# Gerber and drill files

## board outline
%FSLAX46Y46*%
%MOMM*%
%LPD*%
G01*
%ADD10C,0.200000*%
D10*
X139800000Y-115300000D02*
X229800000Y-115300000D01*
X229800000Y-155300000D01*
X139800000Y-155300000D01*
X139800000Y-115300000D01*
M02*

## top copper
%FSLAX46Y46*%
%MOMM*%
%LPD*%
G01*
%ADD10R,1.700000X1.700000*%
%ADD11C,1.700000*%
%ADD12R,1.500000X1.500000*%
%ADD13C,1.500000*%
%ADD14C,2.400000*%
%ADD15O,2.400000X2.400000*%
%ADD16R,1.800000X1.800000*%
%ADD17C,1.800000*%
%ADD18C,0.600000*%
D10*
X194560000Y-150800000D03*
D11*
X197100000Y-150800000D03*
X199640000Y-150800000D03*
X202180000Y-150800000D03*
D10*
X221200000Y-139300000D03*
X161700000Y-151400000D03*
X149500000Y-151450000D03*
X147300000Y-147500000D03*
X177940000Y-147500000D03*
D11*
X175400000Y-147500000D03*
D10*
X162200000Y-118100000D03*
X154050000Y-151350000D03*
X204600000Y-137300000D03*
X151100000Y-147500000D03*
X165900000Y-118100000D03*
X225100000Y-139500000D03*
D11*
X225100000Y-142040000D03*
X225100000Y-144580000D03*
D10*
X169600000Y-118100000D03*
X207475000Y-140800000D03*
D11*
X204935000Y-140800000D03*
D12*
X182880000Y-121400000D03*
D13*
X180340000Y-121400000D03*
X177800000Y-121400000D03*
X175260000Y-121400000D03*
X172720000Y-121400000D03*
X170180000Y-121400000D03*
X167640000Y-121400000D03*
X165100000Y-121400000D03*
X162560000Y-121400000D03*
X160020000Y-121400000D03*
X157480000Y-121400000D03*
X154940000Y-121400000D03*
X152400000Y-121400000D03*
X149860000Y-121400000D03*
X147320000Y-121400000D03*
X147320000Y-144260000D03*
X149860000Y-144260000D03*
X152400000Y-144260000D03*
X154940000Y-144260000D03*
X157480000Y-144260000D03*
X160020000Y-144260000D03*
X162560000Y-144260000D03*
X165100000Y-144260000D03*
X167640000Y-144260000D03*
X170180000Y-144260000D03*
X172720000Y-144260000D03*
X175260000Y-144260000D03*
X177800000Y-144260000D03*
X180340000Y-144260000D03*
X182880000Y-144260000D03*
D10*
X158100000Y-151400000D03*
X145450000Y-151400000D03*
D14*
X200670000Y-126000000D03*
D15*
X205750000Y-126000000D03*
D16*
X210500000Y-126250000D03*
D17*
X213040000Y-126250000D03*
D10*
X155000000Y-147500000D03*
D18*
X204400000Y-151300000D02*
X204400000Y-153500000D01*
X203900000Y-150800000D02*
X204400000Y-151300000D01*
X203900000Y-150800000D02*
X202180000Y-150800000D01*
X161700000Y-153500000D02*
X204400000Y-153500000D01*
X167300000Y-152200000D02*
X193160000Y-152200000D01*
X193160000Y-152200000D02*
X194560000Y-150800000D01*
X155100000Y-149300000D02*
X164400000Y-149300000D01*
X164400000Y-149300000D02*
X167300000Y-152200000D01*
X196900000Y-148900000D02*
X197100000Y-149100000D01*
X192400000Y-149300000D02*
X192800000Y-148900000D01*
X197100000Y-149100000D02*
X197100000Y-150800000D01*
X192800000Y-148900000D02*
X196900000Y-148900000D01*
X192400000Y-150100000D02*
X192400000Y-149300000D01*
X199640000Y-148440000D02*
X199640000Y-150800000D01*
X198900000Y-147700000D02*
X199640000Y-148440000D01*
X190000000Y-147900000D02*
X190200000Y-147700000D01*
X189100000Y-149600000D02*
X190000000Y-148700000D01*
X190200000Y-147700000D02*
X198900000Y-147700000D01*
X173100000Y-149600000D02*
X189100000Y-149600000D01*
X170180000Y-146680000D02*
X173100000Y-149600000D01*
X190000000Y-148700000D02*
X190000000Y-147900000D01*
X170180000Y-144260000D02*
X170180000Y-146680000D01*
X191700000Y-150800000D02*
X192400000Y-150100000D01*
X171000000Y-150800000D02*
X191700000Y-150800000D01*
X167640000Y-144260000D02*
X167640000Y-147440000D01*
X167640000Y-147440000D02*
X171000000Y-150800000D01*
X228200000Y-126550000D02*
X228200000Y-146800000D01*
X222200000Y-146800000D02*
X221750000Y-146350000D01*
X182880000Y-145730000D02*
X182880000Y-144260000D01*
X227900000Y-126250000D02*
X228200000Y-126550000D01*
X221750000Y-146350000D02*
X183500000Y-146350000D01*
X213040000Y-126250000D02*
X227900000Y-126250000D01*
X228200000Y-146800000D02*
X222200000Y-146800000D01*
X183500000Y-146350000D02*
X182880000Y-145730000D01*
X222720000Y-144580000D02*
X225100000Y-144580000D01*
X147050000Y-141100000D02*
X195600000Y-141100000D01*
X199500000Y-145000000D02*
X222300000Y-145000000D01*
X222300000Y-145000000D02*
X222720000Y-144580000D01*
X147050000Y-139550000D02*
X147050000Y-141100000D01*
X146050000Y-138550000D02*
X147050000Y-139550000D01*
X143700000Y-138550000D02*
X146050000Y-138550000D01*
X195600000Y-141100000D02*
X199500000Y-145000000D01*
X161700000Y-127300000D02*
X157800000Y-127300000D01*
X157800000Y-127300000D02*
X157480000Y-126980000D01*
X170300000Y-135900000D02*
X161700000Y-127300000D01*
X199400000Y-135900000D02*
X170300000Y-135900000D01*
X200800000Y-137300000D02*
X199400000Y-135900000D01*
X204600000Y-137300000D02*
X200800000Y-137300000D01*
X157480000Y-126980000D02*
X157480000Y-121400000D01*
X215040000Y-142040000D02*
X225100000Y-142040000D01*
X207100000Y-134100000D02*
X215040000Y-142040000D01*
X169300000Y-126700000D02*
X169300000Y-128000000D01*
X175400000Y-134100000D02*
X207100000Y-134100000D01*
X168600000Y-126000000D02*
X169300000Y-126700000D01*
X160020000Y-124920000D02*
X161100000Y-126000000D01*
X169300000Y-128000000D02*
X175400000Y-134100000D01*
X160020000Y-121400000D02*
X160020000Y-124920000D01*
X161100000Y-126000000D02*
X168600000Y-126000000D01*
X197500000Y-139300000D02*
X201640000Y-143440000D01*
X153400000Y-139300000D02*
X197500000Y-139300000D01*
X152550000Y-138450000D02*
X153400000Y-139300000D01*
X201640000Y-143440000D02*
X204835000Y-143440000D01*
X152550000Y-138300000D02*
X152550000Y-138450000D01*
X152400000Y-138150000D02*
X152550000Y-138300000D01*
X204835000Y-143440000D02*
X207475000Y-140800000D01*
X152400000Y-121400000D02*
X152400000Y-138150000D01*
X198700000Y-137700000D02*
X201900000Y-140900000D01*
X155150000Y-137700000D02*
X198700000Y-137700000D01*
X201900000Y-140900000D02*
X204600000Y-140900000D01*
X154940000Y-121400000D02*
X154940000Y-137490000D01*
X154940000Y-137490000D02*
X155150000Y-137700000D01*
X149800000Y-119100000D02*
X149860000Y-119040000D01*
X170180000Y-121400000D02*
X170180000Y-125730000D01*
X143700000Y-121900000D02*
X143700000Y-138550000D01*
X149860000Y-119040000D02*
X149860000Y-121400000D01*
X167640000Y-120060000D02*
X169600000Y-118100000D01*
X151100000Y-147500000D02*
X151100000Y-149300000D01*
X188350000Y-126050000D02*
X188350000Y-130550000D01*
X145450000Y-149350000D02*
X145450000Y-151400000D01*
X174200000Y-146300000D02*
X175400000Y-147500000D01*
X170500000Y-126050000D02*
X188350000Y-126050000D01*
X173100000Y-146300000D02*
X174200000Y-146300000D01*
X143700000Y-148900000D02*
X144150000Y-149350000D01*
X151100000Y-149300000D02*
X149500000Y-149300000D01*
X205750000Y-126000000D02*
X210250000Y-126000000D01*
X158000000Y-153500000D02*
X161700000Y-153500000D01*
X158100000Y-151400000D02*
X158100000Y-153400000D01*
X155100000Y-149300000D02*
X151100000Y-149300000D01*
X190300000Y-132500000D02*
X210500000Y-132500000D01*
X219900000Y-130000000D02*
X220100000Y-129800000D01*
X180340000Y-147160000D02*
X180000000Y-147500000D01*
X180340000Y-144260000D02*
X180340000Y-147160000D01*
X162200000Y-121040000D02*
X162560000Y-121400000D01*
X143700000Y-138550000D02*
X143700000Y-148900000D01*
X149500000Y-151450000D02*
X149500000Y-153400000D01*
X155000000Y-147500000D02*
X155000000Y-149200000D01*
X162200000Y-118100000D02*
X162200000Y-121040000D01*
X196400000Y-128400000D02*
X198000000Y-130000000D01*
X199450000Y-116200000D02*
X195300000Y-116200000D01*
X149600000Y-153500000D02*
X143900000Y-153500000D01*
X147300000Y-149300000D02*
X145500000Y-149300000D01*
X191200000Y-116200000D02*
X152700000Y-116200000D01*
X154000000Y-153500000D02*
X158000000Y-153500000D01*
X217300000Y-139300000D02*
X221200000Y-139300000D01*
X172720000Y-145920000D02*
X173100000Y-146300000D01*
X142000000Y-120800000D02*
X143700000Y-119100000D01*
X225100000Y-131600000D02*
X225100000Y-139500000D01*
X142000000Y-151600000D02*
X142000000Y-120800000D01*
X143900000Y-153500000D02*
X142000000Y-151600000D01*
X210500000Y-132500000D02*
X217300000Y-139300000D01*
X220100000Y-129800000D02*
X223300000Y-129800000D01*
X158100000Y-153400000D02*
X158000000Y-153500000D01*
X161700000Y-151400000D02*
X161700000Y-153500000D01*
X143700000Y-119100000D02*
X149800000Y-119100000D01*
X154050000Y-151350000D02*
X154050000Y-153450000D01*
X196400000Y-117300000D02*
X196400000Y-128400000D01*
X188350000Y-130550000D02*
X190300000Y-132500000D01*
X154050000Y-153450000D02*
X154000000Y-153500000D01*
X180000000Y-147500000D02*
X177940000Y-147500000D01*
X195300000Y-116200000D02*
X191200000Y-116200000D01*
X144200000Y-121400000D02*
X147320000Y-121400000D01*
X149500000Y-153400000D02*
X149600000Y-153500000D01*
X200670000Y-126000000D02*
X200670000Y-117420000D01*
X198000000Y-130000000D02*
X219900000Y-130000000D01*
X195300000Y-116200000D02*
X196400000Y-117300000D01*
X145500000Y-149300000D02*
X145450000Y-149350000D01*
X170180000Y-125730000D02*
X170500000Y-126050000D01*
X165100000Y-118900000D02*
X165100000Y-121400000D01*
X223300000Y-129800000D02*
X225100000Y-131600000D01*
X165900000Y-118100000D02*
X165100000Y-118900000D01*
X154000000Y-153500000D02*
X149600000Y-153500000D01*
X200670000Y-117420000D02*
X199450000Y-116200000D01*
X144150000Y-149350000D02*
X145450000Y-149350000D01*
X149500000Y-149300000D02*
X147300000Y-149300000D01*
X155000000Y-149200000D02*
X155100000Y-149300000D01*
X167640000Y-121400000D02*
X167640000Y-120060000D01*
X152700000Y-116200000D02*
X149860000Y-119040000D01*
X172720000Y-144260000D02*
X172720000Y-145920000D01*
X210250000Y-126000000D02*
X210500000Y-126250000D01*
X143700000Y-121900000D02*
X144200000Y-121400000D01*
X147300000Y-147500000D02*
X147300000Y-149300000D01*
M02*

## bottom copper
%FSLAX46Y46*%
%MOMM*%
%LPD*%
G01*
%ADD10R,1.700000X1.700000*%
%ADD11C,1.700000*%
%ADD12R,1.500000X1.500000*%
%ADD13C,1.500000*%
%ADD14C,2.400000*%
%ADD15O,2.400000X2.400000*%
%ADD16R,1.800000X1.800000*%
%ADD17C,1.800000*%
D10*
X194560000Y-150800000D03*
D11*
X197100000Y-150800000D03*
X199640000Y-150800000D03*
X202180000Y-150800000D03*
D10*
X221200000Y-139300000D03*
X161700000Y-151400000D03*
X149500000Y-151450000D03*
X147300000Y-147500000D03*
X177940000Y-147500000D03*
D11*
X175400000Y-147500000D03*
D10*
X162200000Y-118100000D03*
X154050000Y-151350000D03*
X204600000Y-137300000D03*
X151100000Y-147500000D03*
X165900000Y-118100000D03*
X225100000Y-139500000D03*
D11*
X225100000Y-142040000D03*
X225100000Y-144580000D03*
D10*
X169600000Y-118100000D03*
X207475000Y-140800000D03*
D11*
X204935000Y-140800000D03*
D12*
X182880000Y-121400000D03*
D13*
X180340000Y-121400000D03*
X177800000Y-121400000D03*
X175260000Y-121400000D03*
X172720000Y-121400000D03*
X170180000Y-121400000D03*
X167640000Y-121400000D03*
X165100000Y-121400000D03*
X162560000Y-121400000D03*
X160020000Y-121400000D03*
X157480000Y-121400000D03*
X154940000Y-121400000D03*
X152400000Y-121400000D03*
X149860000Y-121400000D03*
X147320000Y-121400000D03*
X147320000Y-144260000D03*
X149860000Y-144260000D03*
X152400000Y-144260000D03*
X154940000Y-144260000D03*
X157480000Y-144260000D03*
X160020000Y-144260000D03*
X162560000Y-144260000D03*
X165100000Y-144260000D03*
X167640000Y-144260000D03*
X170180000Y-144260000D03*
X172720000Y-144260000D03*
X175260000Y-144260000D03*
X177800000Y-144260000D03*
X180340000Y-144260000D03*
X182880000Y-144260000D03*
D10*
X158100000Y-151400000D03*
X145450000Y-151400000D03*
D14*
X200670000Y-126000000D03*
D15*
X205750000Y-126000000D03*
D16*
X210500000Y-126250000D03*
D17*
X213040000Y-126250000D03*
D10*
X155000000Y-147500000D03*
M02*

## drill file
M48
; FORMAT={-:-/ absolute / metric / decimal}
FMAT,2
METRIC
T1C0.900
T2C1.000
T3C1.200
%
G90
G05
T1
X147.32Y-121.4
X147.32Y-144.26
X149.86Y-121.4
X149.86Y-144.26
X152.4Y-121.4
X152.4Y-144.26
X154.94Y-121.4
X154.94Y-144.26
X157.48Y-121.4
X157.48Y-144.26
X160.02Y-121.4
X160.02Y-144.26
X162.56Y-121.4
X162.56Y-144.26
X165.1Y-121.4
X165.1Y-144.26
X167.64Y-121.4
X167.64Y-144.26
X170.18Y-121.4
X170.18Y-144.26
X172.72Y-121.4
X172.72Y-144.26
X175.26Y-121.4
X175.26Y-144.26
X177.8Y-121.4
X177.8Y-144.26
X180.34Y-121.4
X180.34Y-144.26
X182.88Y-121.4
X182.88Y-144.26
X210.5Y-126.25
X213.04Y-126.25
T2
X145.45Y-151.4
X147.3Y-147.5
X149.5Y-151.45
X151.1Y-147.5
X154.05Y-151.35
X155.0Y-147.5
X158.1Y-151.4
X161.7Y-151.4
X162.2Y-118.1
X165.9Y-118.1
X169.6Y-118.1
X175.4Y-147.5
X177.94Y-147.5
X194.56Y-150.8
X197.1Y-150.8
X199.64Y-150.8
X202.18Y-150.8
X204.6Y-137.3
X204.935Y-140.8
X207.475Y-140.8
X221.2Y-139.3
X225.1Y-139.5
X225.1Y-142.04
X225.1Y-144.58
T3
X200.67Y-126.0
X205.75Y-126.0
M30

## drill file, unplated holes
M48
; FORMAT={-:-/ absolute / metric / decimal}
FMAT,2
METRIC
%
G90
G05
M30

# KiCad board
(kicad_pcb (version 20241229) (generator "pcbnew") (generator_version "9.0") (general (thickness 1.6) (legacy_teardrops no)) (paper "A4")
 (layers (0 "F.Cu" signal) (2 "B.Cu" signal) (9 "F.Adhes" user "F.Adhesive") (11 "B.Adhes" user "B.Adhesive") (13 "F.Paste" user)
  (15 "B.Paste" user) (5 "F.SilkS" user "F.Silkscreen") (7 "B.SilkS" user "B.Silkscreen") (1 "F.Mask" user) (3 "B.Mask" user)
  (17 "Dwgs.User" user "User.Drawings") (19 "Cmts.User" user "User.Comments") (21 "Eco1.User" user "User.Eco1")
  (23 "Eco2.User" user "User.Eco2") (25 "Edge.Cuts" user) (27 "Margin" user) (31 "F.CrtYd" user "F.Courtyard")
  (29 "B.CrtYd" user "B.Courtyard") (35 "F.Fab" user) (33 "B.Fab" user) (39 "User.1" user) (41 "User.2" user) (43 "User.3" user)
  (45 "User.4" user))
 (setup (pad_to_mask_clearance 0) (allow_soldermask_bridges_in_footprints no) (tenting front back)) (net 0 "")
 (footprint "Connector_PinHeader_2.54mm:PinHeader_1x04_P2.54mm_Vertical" (layer "F.Cu") (at 194.56 150.8 90)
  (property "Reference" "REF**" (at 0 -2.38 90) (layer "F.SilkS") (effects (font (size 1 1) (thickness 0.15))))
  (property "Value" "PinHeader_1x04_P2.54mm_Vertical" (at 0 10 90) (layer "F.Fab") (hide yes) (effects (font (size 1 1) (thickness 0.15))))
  (pad "1" thru_hole rect (at 0 0 90) (size 1.7 1.7) (drill 1) (layers "*.Cu" "*.Mask") (remove_unused_layers no))
  (pad "2" thru_hole circle (at 0 2.54 90) (size 1.7 1.7) (drill 1) (layers "*.Cu" "*.Mask") (remove_unused_layers no))
  (pad "3" thru_hole circle (at 0 5.08 90) (size 1.7 1.7) (drill 1) (layers "*.Cu" "*.Mask") (remove_unused_layers no))
  (pad "4" thru_hole circle (at 0 7.62 90) (size 1.7 1.7) (drill 1) (layers "*.Cu" "*.Mask") (remove_unused_layers no)))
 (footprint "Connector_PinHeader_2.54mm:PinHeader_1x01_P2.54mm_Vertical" (layer "F.Cu") (at 221.2 139.3 90)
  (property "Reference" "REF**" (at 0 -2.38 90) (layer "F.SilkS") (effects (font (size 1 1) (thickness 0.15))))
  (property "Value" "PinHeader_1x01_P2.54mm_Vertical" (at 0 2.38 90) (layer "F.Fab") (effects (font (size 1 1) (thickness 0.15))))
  (pad "1" thru_hole rect (at 0 0 90) (size 1.7 1.7) (drill 1) (layers "*.Cu" "*.Mask") (remove_unused_layers no)))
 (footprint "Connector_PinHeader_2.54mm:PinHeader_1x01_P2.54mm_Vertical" (layer "F.Cu") (at 161.7 151.4)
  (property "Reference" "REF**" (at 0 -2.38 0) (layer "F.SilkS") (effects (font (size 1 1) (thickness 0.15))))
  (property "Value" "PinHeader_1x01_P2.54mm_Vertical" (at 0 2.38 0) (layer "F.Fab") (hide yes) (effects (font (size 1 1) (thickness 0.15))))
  (pad "1" thru_hole rect (at 0 0) (size 1.7 1.7) (drill 1) (layers "*.Cu" "*.Mask") (remove_unused_layers no)))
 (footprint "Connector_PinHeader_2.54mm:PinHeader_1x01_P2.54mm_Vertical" (layer "F.Cu") (at 149.5 151.45)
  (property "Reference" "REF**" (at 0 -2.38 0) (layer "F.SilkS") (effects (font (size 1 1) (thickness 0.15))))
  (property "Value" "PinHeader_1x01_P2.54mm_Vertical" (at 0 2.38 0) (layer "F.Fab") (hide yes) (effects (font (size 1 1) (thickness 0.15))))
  (pad "1" thru_hole rect (at 0 0) (size 1.7 1.7) (drill 1) (layers "*.Cu" "*.Mask") (remove_unused_layers no)))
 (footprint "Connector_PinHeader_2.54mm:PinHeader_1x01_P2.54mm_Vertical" (layer "F.Cu") (at 147.3 147.5)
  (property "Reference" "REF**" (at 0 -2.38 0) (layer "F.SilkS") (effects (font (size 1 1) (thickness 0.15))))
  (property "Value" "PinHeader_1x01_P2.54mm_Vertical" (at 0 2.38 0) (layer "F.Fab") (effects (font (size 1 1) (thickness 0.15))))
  (pad "1" thru_hole rect (at 0 0) (size 1.7 1.7) (drill 1) (layers "*.Cu" "*.Mask") (remove_unused_layers no)))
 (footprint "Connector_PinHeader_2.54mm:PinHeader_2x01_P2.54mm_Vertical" (layer "F.Cu") (at 177.94 147.5 180)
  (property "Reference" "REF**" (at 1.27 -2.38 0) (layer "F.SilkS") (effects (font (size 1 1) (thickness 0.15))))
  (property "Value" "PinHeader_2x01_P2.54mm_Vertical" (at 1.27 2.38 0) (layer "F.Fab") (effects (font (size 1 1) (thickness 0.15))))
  (pad "1" thru_hole rect (at 0 0 180) (size 1.7 1.7) (drill 1) (layers "*.Cu" "*.Mask") (remove_unused_layers no))
  (pad "2" thru_hole circle (at 2.54 0 180) (size 1.7 1.7) (drill 1) (layers "*.Cu" "*.Mask") (remove_unused_layers no)))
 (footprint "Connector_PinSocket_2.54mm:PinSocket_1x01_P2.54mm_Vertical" (layer "F.Cu") (at 162.2 118.1)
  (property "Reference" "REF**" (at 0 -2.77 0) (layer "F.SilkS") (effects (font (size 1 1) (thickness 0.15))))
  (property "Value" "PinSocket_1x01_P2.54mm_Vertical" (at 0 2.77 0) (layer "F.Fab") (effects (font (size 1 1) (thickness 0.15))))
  (pad "1" thru_hole rect (at 0 0) (size 1.7 1.7) (drill 1) (layers "*.Cu" "*.Mask") (remove_unused_layers no)))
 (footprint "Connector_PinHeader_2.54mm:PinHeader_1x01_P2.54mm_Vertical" (layer "F.Cu") (at 154.05 151.35 -90)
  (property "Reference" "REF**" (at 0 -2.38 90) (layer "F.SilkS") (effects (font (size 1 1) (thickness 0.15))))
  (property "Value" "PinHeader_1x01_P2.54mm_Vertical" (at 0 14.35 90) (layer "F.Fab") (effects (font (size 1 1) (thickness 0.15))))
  (pad "1" thru_hole rect (at 0 0 270) (size 1.7 1.7) (drill 1) (layers "*.Cu" "*.Mask") (remove_unused_layers no)))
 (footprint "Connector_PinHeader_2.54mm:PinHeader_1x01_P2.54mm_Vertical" (layer "F.Cu") (at 204.6 137.3 90)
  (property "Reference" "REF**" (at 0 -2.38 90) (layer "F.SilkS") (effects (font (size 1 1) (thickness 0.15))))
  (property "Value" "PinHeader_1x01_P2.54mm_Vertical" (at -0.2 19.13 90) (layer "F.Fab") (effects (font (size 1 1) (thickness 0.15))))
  (pad "1" thru_hole rect (at 0 0 90) (size 1.7 1.7) (drill 1) (layers "*.Cu" "*.Mask") (remove_unused_layers no)))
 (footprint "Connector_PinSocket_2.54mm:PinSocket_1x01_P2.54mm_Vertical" (layer "F.Cu") (at 151.1 147.5)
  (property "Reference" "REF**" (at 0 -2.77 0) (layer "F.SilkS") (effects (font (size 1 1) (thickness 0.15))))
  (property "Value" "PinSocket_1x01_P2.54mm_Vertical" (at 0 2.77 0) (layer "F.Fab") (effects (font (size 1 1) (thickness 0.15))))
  (pad "1" thru_hole rect (at 0 0) (size 1.7 1.7) (drill 1) (layers "*.Cu" "*.Mask") (remove_unused_layers no)))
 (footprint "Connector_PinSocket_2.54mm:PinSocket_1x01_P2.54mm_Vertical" (layer "F.Cu") (at 165.9 118.1)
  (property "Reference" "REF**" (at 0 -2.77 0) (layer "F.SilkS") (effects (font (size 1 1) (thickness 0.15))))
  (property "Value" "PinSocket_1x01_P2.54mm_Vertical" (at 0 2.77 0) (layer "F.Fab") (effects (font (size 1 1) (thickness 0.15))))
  (pad "1" thru_hole rect (at 0 0) (size 1.7 1.7) (drill 1) (layers "*.Cu" "*.Mask") (remove_unused_layers no)))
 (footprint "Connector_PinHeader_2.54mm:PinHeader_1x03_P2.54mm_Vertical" (layer "F.Cu") (at 225.1 139.5)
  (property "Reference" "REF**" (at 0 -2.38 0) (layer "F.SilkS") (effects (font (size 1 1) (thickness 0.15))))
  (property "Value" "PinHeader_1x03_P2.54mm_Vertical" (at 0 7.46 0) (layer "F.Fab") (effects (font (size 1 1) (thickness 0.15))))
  (pad "1" thru_hole rect (at 0 0) (size 1.7 1.7) (drill 1) (layers "*.Cu" "*.Mask") (remove_unused_layers no))
  (pad "2" thru_hole circle (at 0 2.54) (size 1.7 1.7) (drill 1) (layers "*.Cu" "*.Mask") (remove_unused_layers no))
  (pad "3" thru_hole circle (at 0 5.08) (size 1.7 1.7) (drill 1) (layers "*.Cu" "*.Mask") (remove_unused_layers no)))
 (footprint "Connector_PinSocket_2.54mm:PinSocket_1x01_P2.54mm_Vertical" (layer "F.Cu") (at 169.6 118.1)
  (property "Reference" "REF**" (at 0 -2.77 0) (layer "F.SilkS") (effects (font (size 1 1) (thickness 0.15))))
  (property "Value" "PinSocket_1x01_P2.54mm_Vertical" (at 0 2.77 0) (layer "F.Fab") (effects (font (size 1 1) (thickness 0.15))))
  (pad "1" thru_hole rect (at 0 0) (size 1.7 1.7) (drill 1) (layers "*.Cu" "*.Mask") (remove_unused_layers no)))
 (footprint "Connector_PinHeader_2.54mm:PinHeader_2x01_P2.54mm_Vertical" (layer "F.Cu") (at 207.475 140.8 180)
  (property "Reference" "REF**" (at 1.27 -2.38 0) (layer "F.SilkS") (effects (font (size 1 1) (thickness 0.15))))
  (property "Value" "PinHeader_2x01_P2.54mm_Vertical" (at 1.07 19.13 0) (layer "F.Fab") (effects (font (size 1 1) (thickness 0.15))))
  (pad "1" thru_hole rect (at 0 0 180) (size 1.7 1.7) (drill 1) (layers "*.Cu" "*.Mask") (remove_unused_layers no))
  (pad "2" thru_hole circle (at 2.54 0 180) (size 1.7 1.7) (drill 1) (layers "*.Cu" "*.Mask") (remove_unused_layers no)))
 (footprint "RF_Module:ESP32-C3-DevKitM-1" (layer "F.Cu") (at 182.88 121.4 -90)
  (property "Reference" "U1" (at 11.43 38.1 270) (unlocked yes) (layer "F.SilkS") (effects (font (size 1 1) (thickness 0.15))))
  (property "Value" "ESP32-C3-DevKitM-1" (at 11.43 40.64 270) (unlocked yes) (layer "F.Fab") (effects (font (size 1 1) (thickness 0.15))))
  (pad "1" thru_hole rect (at 0 0 270) (size 1.5 1.5) (drill 0.9) (layers "*.Cu" "*.Mask") (remove_unused_layers yes) (keep_end_layers yes)
   (zone_layer_connections))
  (pad "2" thru_hole circle (at 0 2.54 270) (size 1.5 1.5) (drill 0.9) (layers "*.Cu" "*.Mask") (remove_unused_layers yes)
   (keep_end_layers yes) (zone_layer_connections))
  (pad "3" thru_hole circle (at 0 5.08 270) (size 1.5 1.5) (drill 0.9) (layers "*.Cu" "*.Mask") (remove_unused_layers yes)
   (keep_end_layers yes) (zone_layer_connections))
  (pad "4" thru_hole circle (at 0 7.62 270) (size 1.5 1.5) (drill 0.9) (layers "*.Cu" "*.Mask") (remove_unused_layers yes)
   (keep_end_layers yes) (zone_layer_connections))
  (pad "5" thru_hole circle (at 0 10.16 270) (size 1.5 1.5) (drill 0.9) (layers "*.Cu" "*.Mask") (remove_unused_layers yes)
   (keep_end_layers yes) (zone_layer_connections))
  (pad "6" thru_hole circle (at 0 12.7 270) (size 1.5 1.5) (drill 0.9) (layers "*.Cu" "*.Mask") (remove_unused_layers yes)
   (keep_end_layers yes) (zone_layer_connections))
  (pad "7" thru_hole circle (at 0 15.24 270) (size 1.5 1.5) (drill 0.9) (layers "*.Cu" "*.Mask") (remove_unused_layers yes)
   (keep_end_layers yes) (zone_layer_connections))
  (pad "8" thru_hole circle (at 0 17.78 270) (size 1.5 1.5) (drill 0.9) (layers "*.Cu" "*.Mask") (remove_unused_layers yes)
   (keep_end_layers yes) (zone_layer_connections))
  (pad "9" thru_hole circle (at 0 20.32 270) (size 1.5 1.5) (drill 0.9) (layers "*.Cu" "*.Mask") (remove_unused_layers yes)
   (keep_end_layers yes) (zone_layer_connections))
  (pad "10" thru_hole circle (at 0 22.86 270) (size 1.5 1.5) (drill 0.9) (layers "*.Cu" "*.Mask") (remove_unused_layers yes)
   (keep_end_layers yes) (zone_layer_connections))
  (pad "11" thru_hole circle (at 0 25.4 270) (size 1.5 1.5) (drill 0.9) (layers "*.Cu" "*.Mask") (remove_unused_layers yes)
   (keep_end_layers yes) (zone_layer_connections))
  (pad "12" thru_hole circle (at 0 27.94 270) (size 1.5 1.5) (drill 0.9) (layers "*.Cu" "*.Mask") (remove_unused_layers yes)
   (keep_end_layers yes) (zone_layer_connections))
  (pad "13" thru_hole circle (at 0 30.48 270) (size 1.5 1.5) (drill 0.9) (layers "*.Cu" "*.Mask") (remove_unused_layers yes)
   (keep_end_layers yes) (zone_layer_connections))
  (pad "14" thru_hole circle (at 0 33.02 270) (size 1.5 1.5) (drill 0.9) (layers "*.Cu" "*.Mask") (remove_unused_layers yes)
   (keep_end_layers yes) (zone_layer_connections))
  (pad "15" thru_hole circle (at 0 35.56 270) (size 1.5 1.5) (drill 0.9) (layers "*.Cu" "*.Mask") (remove_unused_layers yes)
   (keep_end_layers yes) (zone_layer_connections))
  (pad "16" thru_hole circle (at 22.86 35.56 270) (size 1.5 1.5) (drill 0.9) (layers "*.Cu" "*.Mask") (remove_unused_layers yes)
   (keep_end_layers yes) (zone_layer_connections))
  (pad "17" thru_hole circle (at 22.86 33.02 270) (size 1.5 1.5) (drill 0.9) (layers "*.Cu" "*.Mask") (remove_unused_layers yes)
   (keep_end_layers yes) (zone_layer_connections))
  (pad "18" thru_hole circle (at 22.86 30.48 270) (size 1.5 1.5) (drill 0.9) (layers "*.Cu" "*.Mask") (remove_unused_layers yes)
   (keep_end_layers yes) (zone_layer_connections))
  (pad "19" thru_hole circle (at 22.86 27.94 270) (size 1.5 1.5) (drill 0.9) (layers "*.Cu" "*.Mask") (remove_unused_layers yes)
   (keep_end_layers yes) (zone_layer_connections))
  (pad "20" thru_hole circle (at 22.86 25.4 270) (size 1.5 1.5) (drill 0.9) (layers "*.Cu" "*.Mask") (remove_unused_layers yes)
   (keep_end_layers yes) (zone_layer_connections))
  (pad "21" thru_hole circle (at 22.86 22.86 270) (size 1.5 1.5) (drill 0.9) (layers "*.Cu" "*.Mask") (remove_unused_layers yes)
   (keep_end_layers yes) (zone_layer_connections))
  (pad "22" thru_hole circle (at 22.86 20.32 270) (size 1.5 1.5) (drill 0.9) (layers "*.Cu" "*.Mask") (remove_unused_layers yes)
   (keep_end_layers yes) (zone_layer_connections))
  (pad "23" thru_hole circle (at 22.86 17.78 270) (size 1.5 1.5) (drill 0.9) (layers "*.Cu" "*.Mask") (remove_unused_layers yes)
   (keep_end_layers yes) (zone_layer_connections))
  (pad "24" thru_hole circle (at 22.86 15.24 270) (size 1.5 1.5) (drill 0.9) (layers "*.Cu" "*.Mask") (remove_unused_layers yes)
   (keep_end_layers yes) (zone_layer_connections))
  (pad "25" thru_hole circle (at 22.86 12.7 270) (size 1.5 1.5) (drill 0.9) (layers "*.Cu" "*.Mask") (remove_unused_layers yes)
   (keep_end_layers yes) (zone_layer_connections))
  (pad "26" thru_hole circle (at 22.86 10.16 270) (size 1.5 1.5) (drill 0.9) (layers "*.Cu" "*.Mask") (remove_unused_layers yes)
   (keep_end_layers yes) (zone_layer_connections))
  (pad "27" thru_hole circle (at 22.86 7.62 270) (size 1.5 1.5) (drill 0.9) (layers "*.Cu" "*.Mask") (remove_unused_layers yes)
   (keep_end_layers yes) (zone_layer_connections))
  (pad "28" thru_hole circle (at 22.86 5.08 270) (size 1.5 1.5) (drill 0.9) (layers "*.Cu" "*.Mask") (remove_unused_layers yes)
   (keep_end_layers yes) (zone_layer_connections))
  (pad "29" thru_hole circle (at 22.86 2.54 270) (size 1.5 1.5) (drill 0.9) (layers "*.Cu" "*.Mask") (remove_unused_layers yes)
   (keep_end_layers yes) (zone_layer_connections))
  (pad "30" thru_hole circle (at 22.86 0 270) (size 1.5 1.5) (drill 0.9) (layers "*.Cu" "*.Mask") (remove_unused_layers yes)
   (keep_end_layers yes) (zone_layer_connections)))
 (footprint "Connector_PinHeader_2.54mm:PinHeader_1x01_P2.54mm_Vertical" (layer "F.Cu") (at 158.1 151.4)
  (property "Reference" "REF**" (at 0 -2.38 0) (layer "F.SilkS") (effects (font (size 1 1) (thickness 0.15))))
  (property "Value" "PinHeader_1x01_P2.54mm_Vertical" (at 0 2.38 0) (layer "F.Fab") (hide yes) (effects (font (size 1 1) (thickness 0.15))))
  (pad "1" thru_hole rect (at 0 0) (size 1.7 1.7) (drill 1) (layers "*.Cu" "*.Mask") (remove_unused_layers no)))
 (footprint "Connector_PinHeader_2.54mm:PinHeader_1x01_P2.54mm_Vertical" (layer "F.Cu") (at 145.45 151.4 -90)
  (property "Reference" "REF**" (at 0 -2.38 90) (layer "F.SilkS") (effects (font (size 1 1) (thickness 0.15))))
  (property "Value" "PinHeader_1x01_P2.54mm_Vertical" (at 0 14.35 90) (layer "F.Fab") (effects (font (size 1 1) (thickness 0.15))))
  (pad "1" thru_hole rect (at 0 0 270) (size 1.7 1.7) (drill 1) (layers "*.Cu" "*.Mask") (remove_unused_layers no)))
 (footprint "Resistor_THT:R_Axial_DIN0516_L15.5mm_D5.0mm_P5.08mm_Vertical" (layer "F.Cu") (at 200.67 126)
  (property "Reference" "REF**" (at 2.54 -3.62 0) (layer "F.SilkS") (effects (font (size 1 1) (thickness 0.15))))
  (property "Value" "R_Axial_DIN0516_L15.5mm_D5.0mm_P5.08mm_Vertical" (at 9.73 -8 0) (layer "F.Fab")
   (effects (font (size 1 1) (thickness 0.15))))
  (pad "1" thru_hole circle (at 0 0) (size 2.4 2.4) (drill 1.2) (layers "*.Cu" "*.Mask") (remove_unused_layers no))
  (pad "2" thru_hole oval (at 5.08 0) (size 2.4 2.4) (drill 1.2) (layers "*.Cu" "*.Mask") (remove_unused_layers no)))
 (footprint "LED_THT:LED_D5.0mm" (layer "F.Cu") (at 210.5 126.25)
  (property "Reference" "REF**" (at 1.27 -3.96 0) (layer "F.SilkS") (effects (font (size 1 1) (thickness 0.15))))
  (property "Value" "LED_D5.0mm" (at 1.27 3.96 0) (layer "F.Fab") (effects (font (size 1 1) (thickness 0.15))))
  (pad "1" thru_hole rect (at 0 0) (size 1.8 1.8) (drill 0.9) (layers "*.Cu" "*.Mask") (remove_unused_layers no))
  (pad "2" thru_hole circle (at 2.54 0) (size 1.8 1.8) (drill 0.9) (layers "*.Cu" "*.Mask") (remove_unused_layers no)))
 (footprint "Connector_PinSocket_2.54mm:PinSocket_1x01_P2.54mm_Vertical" (layer "F.Cu") (at 155 147.5)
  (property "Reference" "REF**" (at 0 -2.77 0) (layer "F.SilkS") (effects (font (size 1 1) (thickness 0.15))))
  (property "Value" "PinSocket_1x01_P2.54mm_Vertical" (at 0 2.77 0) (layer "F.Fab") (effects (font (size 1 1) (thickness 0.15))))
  (pad "1" thru_hole rect (at 0 0) (size 1.7 1.7) (drill 1) (layers "*.Cu" "*.Mask") (remove_unused_layers no)))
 (gr_rect (start 139.8 115.3) (end 229.8 155.3) (stroke (width 0.2) (type solid)) (fill no) (layer "Edge.Cuts"))
 (segment (start 149.8 119.1) (end 149.86 119.04) (width 0.6) (layer "F.Cu") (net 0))
 (segment (start 155.15 137.7) (end 198.7 137.7) (width 0.6) (layer "F.Cu") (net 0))
 (segment (start 190 148.7) (end 190 147.9) (width 0.6) (layer "F.Cu") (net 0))
 (segment (start 170.18 121.4) (end 170.18 125.73) (width 0.6) (layer "F.Cu") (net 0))
 (segment (start 228.2 146.8) (end 222.2 146.8) (width 0.6) (layer "F.Cu") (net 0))
 (segment (start 143.7 121.9) (end 143.7 138.55) (width 0.6) (layer "F.Cu") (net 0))
 (segment (start 149.86 119.04) (end 149.86 121.4) (width 0.6) (layer "F.Cu") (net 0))
 (segment (start 167.64 120.06) (end 169.6 118.1) (width 0.6) (layer "F.Cu") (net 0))
 (segment (start 228.2 126.55) (end 228.2 146.8) (width 0.6) (layer "F.Cu") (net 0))
 (segment (start 160.02 124.92) (end 161.1 126) (width 0.6) (layer "F.Cu") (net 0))
 (segment (start 164.4 149.3) (end 167.3 152.2) (width 0.6) (layer "F.Cu") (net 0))
 (segment (start 169.3 128) (end 175.4 134.1) (width 0.6) (layer "F.Cu") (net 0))
 (segment (start 183.5 146.35) (end 182.88 145.73) (width 0.6) (layer "F.Cu") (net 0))
 (segment (start 168.6 126) (end 169.3 126.7) (width 0.6) (layer "F.Cu") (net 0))
 (segment (start 170.18 146.68) (end 173.1 149.6) (width 0.6) (layer "F.Cu") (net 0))
 (segment (start 151.1 147.5) (end 151.1 149.3) (width 0.6) (layer "F.Cu") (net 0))
 (segment (start 188.35 126.05) (end 188.35 130.55) (width 0.6) (layer "F.Cu") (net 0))
 (segment (start 193.16 152.2) (end 194.56 150.8) (width 0.6) (layer "F.Cu") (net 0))
 (segment (start 153.4 139.3) (end 197.5 139.3) (width 0.6) (layer "F.Cu") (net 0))
 (segment (start 145.45 149.35) (end 145.45 151.4) (width 0.6) (layer "F.Cu") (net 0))
 (segment (start 147.05 141.1) (end 195.6 141.1) (width 0.6) (layer "F.Cu") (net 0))
 (segment (start 174.2 146.3) (end 175.4 147.5) (width 0.6) (layer "F.Cu") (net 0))
 (segment (start 199.5 145) (end 222.3 145) (width 0.6) (layer "F.Cu") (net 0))
 (segment (start 203.9 150.8) (end 202.18 150.8) (width 0.6) (layer "F.Cu") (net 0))
 (segment (start 170.5 126.05) (end 188.35 126.05) (width 0.6) (layer "F.Cu") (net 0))
 (segment (start 173.1 146.3) (end 174.2 146.3) (width 0.6) (layer "F.Cu") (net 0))
 (segment (start 143.7 148.9) (end 144.15 149.35) (width 0.6) (layer "F.Cu") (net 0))
 (segment (start 195.6 141.1) (end 199.5 145) (width 0.6) (layer "F.Cu") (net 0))
 (segment (start 189.1 149.6) (end 190 148.7) (width 0.6) (layer "F.Cu") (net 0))
 (segment (start 151.1 149.3) (end 149.5 149.3) (width 0.6) (layer "F.Cu") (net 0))
 (segment (start 200.8 137.3) (end 199.4 135.9) (width 0.6) (layer "F.Cu") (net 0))
 (segment (start 205.75 126) (end 210.25 126) (width 0.6) (layer "F.Cu") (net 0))
 (segment (start 169.3 126.7) (end 169.3 128) (width 0.6) (layer "F.Cu") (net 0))
 (segment (start 158 153.5) (end 161.7 153.5) (width 0.6) (layer "F.Cu") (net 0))
 (segment (start 158.1 151.4) (end 158.1 153.4) (width 0.6) (layer "F.Cu") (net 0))
 (segment (start 175.4 134.1) (end 207.1 134.1) (width 0.6) (layer "F.Cu") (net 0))
 (segment (start 196.9 148.9) (end 197.1 149.1) (width 0.6) (layer "F.Cu") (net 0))
 (segment (start 155.1 149.3) (end 151.1 149.3) (width 0.6) (layer "F.Cu") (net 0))
 (segment (start 171 150.8) (end 191.7 150.8) (width 0.6) (layer "F.Cu") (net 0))
 (segment (start 152.55 138.45) (end 153.4 139.3) (width 0.6) (layer "F.Cu") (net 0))
 (segment (start 190.3 132.5) (end 210.5 132.5) (width 0.6) (layer "F.Cu") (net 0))
 (segment (start 161.7 153.5) (end 204.4 153.5) (width 0.6) (layer "F.Cu") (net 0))
 (segment (start 219.9 130) (end 220.1 129.8) (width 0.6) (layer "F.Cu") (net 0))
 (segment (start 152.55 138.3) (end 152.55 138.45) (width 0.6) (layer "F.Cu") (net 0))
 (segment (start 180.34 147.16) (end 180 147.5) (width 0.6) (layer "F.Cu") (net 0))
 (segment (start 161.7 127.3) (end 157.8 127.3) (width 0.6) (layer "F.Cu") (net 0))
 (segment (start 180.34 144.26) (end 180.34 147.16) (width 0.6) (layer "F.Cu") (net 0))
 (segment (start 162.2 121.04) (end 162.56 121.4) (width 0.6) (layer "F.Cu") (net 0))
 (segment (start 201.9 140.9) (end 204.6 140.9) (width 0.6) (layer "F.Cu") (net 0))
 (segment (start 143.7 138.55) (end 143.7 148.9) (width 0.6) (layer "F.Cu") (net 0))
 (segment (start 149.5 151.45) (end 149.5 153.4) (width 0.6) (layer "F.Cu") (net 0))
 (segment (start 155 147.5) (end 155 149.2) (width 0.6) (layer "F.Cu") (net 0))
 (segment (start 167.3 152.2) (end 193.16 152.2) (width 0.6) (layer "F.Cu") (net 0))
 (segment (start 162.2 118.1) (end 162.2 121.04) (width 0.6) (layer "F.Cu") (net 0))
 (segment (start 204.4 151.3) (end 204.4 153.5) (width 0.6) (layer "F.Cu") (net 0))
 (segment (start 154.94 121.4) (end 154.94 137.49) (width 0.6) (layer "F.Cu") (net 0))
 (segment (start 170.18 144.26) (end 170.18 146.68) (width 0.6) (layer "F.Cu") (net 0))
 (segment (start 196.4 128.4) (end 198 130) (width 0.6) (layer "F.Cu") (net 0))
 (segment (start 199.45 116.2) (end 195.3 116.2) (width 0.6) (layer "F.Cu") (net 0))
 (segment (start 149.6 153.5) (end 143.9 153.5) (width 0.6) (layer "F.Cu") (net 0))
 (segment (start 192.4 150.1) (end 192.4 149.3) (width 0.6) (layer "F.Cu") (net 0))
 (segment (start 190 147.9) (end 190.2 147.7) (width 0.6) (layer "F.Cu") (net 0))
 (segment (start 157.48 126.98) (end 157.48 121.4) (width 0.6) (layer "F.Cu") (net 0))
 (segment (start 191.7 150.8) (end 192.4 150.1) (width 0.6) (layer "F.Cu") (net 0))
 (segment (start 147.3 149.3) (end 145.5 149.3) (width 0.6) (layer "F.Cu") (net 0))
 (segment (start 191.2 116.2) (end 152.7 116.2) (width 0.6) (layer "F.Cu") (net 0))
 (segment (start 190.2 147.7) (end 198.9 147.7) (width 0.6) (layer "F.Cu") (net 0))
 (segment (start 173.1 149.6) (end 189.1 149.6) (width 0.6) (layer "F.Cu") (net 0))
 (segment (start 157.8 127.3) (end 157.48 126.98) (width 0.6) (layer "F.Cu") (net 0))
 (segment (start 192.4 149.3) (end 192.8 148.9) (width 0.6) (layer "F.Cu") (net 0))
 (segment (start 204.6 137.3) (end 200.8 137.3) (width 0.6) (layer "F.Cu") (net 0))
 (segment (start 207.1 134.1) (end 215.04 142.04) (width 0.6) (layer "F.Cu") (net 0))
 (segment (start 154 153.5) (end 158 153.5) (width 0.6) (layer "F.Cu") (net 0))
 (segment (start 217.3 139.3) (end 221.2 139.3) (width 0.6) (layer "F.Cu") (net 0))
 (segment (start 152.4 121.4) (end 152.4 138.15) (width 0.6) (layer "F.Cu") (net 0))
 (segment (start 199.64 148.44) (end 199.64 150.8) (width 0.6) (layer "F.Cu") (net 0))
 (segment (start 172.72 145.92) (end 173.1 146.3) (width 0.6) (layer "F.Cu") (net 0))
 (segment (start 142 120.8) (end 143.7 119.1) (width 0.6) (layer "F.Cu") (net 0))
 (segment (start 222.3 145) (end 222.72 144.58) (width 0.6) (layer "F.Cu") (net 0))
 (segment (start 198.9 147.7) (end 199.64 148.44) (width 0.6) (layer "F.Cu") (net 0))
 (segment (start 225.1 131.6) (end 225.1 139.5) (width 0.6) (layer "F.Cu") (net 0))
 (segment (start 222.72 144.58) (end 225.1 144.58) (width 0.6) (layer "F.Cu") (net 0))
 (segment (start 152.4 138.15) (end 152.55 138.3) (width 0.6) (layer "F.Cu") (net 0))
 (segment (start 167.64 144.26) (end 167.64 147.44) (width 0.6) (layer "F.Cu") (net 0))
 (segment (start 142 151.6) (end 142 120.8) (width 0.6) (layer "F.Cu") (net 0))
 (segment (start 215.04 142.04) (end 225.1 142.04) (width 0.6) (layer "F.Cu") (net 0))
 (segment (start 161.1 126) (end 168.6 126) (width 0.6) (layer "F.Cu") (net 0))
 (segment (start 143.9 153.5) (end 142 151.6) (width 0.6) (layer "F.Cu") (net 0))
 (segment (start 197.1 149.1) (end 197.1 150.8) (width 0.6) (layer "F.Cu") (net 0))
 (segment (start 154.94 137.49) (end 155.15 137.7) (width 0.6) (layer "F.Cu") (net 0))
 (segment (start 210.5 132.5) (end 217.3 139.3) (width 0.6) (layer "F.Cu") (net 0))
 (segment (start 220.1 129.8) (end 223.3 129.8) (width 0.6) (layer "F.Cu") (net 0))
 (segment (start 158.1 153.4) (end 158 153.5) (width 0.6) (layer "F.Cu") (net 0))
 (segment (start 227.9 126.25) (end 228.2 126.55) (width 0.6) (layer "F.Cu") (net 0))
 (segment (start 161.7 151.4) (end 161.7 153.5) (width 0.6) (layer "F.Cu") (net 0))
 (segment (start 155.1 149.3) (end 164.4 149.3) (width 0.6) (layer "F.Cu") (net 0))
 (segment (start 143.7 119.1) (end 149.8 119.1) (width 0.6) (layer "F.Cu") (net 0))
 (segment (start 154.05 151.35) (end 154.05 153.45) (width 0.6) (layer "F.Cu") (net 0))
 (segment (start 196.4 117.3) (end 196.4 128.4) (width 0.6) (layer "F.Cu") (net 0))
 (segment (start 188.35 130.55) (end 190.3 132.5) (width 0.6) (layer "F.Cu") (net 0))
 (segment (start 213.04 126.25) (end 227.9 126.25) (width 0.6) (layer "F.Cu") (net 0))
 (segment (start 143.7 138.55) (end 146.05 138.55) (width 0.6) (layer "F.Cu") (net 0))
 (segment (start 154.05 153.45) (end 154 153.5) (width 0.6) (layer "F.Cu") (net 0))
 (segment (start 160.02 121.4) (end 160.02 124.92) (width 0.6) (layer "F.Cu") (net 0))
 (segment (start 180 147.5) (end 177.94 147.5) (width 0.6) (layer "F.Cu") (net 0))
 (segment (start 195.3 116.2) (end 191.2 116.2) (width 0.6) (layer "F.Cu") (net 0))
 (segment (start 201.64 143.44) (end 204.835 143.44) (width 0.6) (layer "F.Cu") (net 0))
 (segment (start 204.835 143.44) (end 207.475 140.8) (width 0.6) (layer "F.Cu") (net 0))
 (segment (start 144.2 121.4) (end 147.32 121.4) (width 0.6) (layer "F.Cu") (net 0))
 (segment (start 167.64 147.44) (end 171 150.8) (width 0.6) (layer "F.Cu") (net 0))
 (segment (start 149.5 153.4) (end 149.6 153.5) (width 0.6) (layer "F.Cu") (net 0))
 (segment (start 197.5 139.3) (end 201.64 143.44) (width 0.6) (layer "F.Cu") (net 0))
 (segment (start 182.88 145.73) (end 182.88 144.26) (width 0.6) (layer "F.Cu") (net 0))
 (segment (start 200.67 126) (end 200.67 117.42) (width 0.6) (layer "F.Cu") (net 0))
 (segment (start 198 130) (end 219.9 130) (width 0.6) (layer "F.Cu") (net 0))
 (segment (start 147.05 139.55) (end 147.05 141.1) (width 0.6) (layer "F.Cu") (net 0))
 (segment (start 195.3 116.2) (end 196.4 117.3) (width 0.6) (layer "F.Cu") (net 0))
 (segment (start 170.3 135.9) (end 161.7 127.3) (width 0.6) (layer "F.Cu") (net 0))
 (segment (start 145.5 149.3) (end 145.45 149.35) (width 0.6) (layer "F.Cu") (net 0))
 (segment (start 170.18 125.73) (end 170.5 126.05) (width 0.6) (layer "F.Cu") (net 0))
 (segment (start 165.1 118.9) (end 165.1 121.4) (width 0.6) (layer "F.Cu") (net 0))
 (segment (start 223.3 129.8) (end 225.1 131.6) (width 0.6) (layer "F.Cu") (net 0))
 (segment (start 165.9 118.1) (end 165.1 118.9) (width 0.6) (layer "F.Cu") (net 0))
 (segment (start 154 153.5) (end 149.6 153.5) (width 0.6) (layer "F.Cu") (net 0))
 (segment (start 200.67 117.42) (end 199.45 116.2) (width 0.6) (layer "F.Cu") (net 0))
 (segment (start 144.15 149.35) (end 145.45 149.35) (width 0.6) (layer "F.Cu") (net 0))
 (segment (start 192.8 148.9) (end 196.9 148.9) (width 0.6) (layer "F.Cu") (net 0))
 (segment (start 149.5 149.3) (end 147.3 149.3) (width 0.6) (layer "F.Cu") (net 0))
 (segment (start 203.9 150.8) (end 204.4 151.3) (width 0.6) (layer "F.Cu") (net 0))
 (segment (start 155 149.2) (end 155.1 149.3) (width 0.6) (layer "F.Cu") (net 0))
 (segment (start 167.64 121.4) (end 167.64 120.06) (width 0.6) (layer "F.Cu") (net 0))
 (segment (start 222.2 146.8) (end 221.75 146.35) (width 0.6) (layer "F.Cu") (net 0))
 (segment (start 152.7 116.2) (end 149.86 119.04) (width 0.6) (layer "F.Cu") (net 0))
 (segment (start 172.72 144.26) (end 172.72 145.92) (width 0.6) (layer "F.Cu") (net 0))
 (segment (start 210.25 126) (end 210.5 126.25) (width 0.6) (layer "F.Cu") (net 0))
 (segment (start 221.75 146.35) (end 183.5 146.35) (width 0.6) (layer "F.Cu") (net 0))
 (segment (start 198.7 137.7) (end 201.9 140.9) (width 0.6) (layer "F.Cu") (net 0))
 (segment (start 199.4 135.9) (end 170.3 135.9) (width 0.6) (layer "F.Cu") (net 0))
 (segment (start 143.7 121.9) (end 144.2 121.4) (width 0.6) (layer "F.Cu") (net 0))
 (segment (start 146.05 138.55) (end 147.05 139.55) (width 0.6) (layer "F.Cu") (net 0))
 (segment (start 147.3 147.5) (end 147.3 149.3) (width 0.6) (layer "F.Cu") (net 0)))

